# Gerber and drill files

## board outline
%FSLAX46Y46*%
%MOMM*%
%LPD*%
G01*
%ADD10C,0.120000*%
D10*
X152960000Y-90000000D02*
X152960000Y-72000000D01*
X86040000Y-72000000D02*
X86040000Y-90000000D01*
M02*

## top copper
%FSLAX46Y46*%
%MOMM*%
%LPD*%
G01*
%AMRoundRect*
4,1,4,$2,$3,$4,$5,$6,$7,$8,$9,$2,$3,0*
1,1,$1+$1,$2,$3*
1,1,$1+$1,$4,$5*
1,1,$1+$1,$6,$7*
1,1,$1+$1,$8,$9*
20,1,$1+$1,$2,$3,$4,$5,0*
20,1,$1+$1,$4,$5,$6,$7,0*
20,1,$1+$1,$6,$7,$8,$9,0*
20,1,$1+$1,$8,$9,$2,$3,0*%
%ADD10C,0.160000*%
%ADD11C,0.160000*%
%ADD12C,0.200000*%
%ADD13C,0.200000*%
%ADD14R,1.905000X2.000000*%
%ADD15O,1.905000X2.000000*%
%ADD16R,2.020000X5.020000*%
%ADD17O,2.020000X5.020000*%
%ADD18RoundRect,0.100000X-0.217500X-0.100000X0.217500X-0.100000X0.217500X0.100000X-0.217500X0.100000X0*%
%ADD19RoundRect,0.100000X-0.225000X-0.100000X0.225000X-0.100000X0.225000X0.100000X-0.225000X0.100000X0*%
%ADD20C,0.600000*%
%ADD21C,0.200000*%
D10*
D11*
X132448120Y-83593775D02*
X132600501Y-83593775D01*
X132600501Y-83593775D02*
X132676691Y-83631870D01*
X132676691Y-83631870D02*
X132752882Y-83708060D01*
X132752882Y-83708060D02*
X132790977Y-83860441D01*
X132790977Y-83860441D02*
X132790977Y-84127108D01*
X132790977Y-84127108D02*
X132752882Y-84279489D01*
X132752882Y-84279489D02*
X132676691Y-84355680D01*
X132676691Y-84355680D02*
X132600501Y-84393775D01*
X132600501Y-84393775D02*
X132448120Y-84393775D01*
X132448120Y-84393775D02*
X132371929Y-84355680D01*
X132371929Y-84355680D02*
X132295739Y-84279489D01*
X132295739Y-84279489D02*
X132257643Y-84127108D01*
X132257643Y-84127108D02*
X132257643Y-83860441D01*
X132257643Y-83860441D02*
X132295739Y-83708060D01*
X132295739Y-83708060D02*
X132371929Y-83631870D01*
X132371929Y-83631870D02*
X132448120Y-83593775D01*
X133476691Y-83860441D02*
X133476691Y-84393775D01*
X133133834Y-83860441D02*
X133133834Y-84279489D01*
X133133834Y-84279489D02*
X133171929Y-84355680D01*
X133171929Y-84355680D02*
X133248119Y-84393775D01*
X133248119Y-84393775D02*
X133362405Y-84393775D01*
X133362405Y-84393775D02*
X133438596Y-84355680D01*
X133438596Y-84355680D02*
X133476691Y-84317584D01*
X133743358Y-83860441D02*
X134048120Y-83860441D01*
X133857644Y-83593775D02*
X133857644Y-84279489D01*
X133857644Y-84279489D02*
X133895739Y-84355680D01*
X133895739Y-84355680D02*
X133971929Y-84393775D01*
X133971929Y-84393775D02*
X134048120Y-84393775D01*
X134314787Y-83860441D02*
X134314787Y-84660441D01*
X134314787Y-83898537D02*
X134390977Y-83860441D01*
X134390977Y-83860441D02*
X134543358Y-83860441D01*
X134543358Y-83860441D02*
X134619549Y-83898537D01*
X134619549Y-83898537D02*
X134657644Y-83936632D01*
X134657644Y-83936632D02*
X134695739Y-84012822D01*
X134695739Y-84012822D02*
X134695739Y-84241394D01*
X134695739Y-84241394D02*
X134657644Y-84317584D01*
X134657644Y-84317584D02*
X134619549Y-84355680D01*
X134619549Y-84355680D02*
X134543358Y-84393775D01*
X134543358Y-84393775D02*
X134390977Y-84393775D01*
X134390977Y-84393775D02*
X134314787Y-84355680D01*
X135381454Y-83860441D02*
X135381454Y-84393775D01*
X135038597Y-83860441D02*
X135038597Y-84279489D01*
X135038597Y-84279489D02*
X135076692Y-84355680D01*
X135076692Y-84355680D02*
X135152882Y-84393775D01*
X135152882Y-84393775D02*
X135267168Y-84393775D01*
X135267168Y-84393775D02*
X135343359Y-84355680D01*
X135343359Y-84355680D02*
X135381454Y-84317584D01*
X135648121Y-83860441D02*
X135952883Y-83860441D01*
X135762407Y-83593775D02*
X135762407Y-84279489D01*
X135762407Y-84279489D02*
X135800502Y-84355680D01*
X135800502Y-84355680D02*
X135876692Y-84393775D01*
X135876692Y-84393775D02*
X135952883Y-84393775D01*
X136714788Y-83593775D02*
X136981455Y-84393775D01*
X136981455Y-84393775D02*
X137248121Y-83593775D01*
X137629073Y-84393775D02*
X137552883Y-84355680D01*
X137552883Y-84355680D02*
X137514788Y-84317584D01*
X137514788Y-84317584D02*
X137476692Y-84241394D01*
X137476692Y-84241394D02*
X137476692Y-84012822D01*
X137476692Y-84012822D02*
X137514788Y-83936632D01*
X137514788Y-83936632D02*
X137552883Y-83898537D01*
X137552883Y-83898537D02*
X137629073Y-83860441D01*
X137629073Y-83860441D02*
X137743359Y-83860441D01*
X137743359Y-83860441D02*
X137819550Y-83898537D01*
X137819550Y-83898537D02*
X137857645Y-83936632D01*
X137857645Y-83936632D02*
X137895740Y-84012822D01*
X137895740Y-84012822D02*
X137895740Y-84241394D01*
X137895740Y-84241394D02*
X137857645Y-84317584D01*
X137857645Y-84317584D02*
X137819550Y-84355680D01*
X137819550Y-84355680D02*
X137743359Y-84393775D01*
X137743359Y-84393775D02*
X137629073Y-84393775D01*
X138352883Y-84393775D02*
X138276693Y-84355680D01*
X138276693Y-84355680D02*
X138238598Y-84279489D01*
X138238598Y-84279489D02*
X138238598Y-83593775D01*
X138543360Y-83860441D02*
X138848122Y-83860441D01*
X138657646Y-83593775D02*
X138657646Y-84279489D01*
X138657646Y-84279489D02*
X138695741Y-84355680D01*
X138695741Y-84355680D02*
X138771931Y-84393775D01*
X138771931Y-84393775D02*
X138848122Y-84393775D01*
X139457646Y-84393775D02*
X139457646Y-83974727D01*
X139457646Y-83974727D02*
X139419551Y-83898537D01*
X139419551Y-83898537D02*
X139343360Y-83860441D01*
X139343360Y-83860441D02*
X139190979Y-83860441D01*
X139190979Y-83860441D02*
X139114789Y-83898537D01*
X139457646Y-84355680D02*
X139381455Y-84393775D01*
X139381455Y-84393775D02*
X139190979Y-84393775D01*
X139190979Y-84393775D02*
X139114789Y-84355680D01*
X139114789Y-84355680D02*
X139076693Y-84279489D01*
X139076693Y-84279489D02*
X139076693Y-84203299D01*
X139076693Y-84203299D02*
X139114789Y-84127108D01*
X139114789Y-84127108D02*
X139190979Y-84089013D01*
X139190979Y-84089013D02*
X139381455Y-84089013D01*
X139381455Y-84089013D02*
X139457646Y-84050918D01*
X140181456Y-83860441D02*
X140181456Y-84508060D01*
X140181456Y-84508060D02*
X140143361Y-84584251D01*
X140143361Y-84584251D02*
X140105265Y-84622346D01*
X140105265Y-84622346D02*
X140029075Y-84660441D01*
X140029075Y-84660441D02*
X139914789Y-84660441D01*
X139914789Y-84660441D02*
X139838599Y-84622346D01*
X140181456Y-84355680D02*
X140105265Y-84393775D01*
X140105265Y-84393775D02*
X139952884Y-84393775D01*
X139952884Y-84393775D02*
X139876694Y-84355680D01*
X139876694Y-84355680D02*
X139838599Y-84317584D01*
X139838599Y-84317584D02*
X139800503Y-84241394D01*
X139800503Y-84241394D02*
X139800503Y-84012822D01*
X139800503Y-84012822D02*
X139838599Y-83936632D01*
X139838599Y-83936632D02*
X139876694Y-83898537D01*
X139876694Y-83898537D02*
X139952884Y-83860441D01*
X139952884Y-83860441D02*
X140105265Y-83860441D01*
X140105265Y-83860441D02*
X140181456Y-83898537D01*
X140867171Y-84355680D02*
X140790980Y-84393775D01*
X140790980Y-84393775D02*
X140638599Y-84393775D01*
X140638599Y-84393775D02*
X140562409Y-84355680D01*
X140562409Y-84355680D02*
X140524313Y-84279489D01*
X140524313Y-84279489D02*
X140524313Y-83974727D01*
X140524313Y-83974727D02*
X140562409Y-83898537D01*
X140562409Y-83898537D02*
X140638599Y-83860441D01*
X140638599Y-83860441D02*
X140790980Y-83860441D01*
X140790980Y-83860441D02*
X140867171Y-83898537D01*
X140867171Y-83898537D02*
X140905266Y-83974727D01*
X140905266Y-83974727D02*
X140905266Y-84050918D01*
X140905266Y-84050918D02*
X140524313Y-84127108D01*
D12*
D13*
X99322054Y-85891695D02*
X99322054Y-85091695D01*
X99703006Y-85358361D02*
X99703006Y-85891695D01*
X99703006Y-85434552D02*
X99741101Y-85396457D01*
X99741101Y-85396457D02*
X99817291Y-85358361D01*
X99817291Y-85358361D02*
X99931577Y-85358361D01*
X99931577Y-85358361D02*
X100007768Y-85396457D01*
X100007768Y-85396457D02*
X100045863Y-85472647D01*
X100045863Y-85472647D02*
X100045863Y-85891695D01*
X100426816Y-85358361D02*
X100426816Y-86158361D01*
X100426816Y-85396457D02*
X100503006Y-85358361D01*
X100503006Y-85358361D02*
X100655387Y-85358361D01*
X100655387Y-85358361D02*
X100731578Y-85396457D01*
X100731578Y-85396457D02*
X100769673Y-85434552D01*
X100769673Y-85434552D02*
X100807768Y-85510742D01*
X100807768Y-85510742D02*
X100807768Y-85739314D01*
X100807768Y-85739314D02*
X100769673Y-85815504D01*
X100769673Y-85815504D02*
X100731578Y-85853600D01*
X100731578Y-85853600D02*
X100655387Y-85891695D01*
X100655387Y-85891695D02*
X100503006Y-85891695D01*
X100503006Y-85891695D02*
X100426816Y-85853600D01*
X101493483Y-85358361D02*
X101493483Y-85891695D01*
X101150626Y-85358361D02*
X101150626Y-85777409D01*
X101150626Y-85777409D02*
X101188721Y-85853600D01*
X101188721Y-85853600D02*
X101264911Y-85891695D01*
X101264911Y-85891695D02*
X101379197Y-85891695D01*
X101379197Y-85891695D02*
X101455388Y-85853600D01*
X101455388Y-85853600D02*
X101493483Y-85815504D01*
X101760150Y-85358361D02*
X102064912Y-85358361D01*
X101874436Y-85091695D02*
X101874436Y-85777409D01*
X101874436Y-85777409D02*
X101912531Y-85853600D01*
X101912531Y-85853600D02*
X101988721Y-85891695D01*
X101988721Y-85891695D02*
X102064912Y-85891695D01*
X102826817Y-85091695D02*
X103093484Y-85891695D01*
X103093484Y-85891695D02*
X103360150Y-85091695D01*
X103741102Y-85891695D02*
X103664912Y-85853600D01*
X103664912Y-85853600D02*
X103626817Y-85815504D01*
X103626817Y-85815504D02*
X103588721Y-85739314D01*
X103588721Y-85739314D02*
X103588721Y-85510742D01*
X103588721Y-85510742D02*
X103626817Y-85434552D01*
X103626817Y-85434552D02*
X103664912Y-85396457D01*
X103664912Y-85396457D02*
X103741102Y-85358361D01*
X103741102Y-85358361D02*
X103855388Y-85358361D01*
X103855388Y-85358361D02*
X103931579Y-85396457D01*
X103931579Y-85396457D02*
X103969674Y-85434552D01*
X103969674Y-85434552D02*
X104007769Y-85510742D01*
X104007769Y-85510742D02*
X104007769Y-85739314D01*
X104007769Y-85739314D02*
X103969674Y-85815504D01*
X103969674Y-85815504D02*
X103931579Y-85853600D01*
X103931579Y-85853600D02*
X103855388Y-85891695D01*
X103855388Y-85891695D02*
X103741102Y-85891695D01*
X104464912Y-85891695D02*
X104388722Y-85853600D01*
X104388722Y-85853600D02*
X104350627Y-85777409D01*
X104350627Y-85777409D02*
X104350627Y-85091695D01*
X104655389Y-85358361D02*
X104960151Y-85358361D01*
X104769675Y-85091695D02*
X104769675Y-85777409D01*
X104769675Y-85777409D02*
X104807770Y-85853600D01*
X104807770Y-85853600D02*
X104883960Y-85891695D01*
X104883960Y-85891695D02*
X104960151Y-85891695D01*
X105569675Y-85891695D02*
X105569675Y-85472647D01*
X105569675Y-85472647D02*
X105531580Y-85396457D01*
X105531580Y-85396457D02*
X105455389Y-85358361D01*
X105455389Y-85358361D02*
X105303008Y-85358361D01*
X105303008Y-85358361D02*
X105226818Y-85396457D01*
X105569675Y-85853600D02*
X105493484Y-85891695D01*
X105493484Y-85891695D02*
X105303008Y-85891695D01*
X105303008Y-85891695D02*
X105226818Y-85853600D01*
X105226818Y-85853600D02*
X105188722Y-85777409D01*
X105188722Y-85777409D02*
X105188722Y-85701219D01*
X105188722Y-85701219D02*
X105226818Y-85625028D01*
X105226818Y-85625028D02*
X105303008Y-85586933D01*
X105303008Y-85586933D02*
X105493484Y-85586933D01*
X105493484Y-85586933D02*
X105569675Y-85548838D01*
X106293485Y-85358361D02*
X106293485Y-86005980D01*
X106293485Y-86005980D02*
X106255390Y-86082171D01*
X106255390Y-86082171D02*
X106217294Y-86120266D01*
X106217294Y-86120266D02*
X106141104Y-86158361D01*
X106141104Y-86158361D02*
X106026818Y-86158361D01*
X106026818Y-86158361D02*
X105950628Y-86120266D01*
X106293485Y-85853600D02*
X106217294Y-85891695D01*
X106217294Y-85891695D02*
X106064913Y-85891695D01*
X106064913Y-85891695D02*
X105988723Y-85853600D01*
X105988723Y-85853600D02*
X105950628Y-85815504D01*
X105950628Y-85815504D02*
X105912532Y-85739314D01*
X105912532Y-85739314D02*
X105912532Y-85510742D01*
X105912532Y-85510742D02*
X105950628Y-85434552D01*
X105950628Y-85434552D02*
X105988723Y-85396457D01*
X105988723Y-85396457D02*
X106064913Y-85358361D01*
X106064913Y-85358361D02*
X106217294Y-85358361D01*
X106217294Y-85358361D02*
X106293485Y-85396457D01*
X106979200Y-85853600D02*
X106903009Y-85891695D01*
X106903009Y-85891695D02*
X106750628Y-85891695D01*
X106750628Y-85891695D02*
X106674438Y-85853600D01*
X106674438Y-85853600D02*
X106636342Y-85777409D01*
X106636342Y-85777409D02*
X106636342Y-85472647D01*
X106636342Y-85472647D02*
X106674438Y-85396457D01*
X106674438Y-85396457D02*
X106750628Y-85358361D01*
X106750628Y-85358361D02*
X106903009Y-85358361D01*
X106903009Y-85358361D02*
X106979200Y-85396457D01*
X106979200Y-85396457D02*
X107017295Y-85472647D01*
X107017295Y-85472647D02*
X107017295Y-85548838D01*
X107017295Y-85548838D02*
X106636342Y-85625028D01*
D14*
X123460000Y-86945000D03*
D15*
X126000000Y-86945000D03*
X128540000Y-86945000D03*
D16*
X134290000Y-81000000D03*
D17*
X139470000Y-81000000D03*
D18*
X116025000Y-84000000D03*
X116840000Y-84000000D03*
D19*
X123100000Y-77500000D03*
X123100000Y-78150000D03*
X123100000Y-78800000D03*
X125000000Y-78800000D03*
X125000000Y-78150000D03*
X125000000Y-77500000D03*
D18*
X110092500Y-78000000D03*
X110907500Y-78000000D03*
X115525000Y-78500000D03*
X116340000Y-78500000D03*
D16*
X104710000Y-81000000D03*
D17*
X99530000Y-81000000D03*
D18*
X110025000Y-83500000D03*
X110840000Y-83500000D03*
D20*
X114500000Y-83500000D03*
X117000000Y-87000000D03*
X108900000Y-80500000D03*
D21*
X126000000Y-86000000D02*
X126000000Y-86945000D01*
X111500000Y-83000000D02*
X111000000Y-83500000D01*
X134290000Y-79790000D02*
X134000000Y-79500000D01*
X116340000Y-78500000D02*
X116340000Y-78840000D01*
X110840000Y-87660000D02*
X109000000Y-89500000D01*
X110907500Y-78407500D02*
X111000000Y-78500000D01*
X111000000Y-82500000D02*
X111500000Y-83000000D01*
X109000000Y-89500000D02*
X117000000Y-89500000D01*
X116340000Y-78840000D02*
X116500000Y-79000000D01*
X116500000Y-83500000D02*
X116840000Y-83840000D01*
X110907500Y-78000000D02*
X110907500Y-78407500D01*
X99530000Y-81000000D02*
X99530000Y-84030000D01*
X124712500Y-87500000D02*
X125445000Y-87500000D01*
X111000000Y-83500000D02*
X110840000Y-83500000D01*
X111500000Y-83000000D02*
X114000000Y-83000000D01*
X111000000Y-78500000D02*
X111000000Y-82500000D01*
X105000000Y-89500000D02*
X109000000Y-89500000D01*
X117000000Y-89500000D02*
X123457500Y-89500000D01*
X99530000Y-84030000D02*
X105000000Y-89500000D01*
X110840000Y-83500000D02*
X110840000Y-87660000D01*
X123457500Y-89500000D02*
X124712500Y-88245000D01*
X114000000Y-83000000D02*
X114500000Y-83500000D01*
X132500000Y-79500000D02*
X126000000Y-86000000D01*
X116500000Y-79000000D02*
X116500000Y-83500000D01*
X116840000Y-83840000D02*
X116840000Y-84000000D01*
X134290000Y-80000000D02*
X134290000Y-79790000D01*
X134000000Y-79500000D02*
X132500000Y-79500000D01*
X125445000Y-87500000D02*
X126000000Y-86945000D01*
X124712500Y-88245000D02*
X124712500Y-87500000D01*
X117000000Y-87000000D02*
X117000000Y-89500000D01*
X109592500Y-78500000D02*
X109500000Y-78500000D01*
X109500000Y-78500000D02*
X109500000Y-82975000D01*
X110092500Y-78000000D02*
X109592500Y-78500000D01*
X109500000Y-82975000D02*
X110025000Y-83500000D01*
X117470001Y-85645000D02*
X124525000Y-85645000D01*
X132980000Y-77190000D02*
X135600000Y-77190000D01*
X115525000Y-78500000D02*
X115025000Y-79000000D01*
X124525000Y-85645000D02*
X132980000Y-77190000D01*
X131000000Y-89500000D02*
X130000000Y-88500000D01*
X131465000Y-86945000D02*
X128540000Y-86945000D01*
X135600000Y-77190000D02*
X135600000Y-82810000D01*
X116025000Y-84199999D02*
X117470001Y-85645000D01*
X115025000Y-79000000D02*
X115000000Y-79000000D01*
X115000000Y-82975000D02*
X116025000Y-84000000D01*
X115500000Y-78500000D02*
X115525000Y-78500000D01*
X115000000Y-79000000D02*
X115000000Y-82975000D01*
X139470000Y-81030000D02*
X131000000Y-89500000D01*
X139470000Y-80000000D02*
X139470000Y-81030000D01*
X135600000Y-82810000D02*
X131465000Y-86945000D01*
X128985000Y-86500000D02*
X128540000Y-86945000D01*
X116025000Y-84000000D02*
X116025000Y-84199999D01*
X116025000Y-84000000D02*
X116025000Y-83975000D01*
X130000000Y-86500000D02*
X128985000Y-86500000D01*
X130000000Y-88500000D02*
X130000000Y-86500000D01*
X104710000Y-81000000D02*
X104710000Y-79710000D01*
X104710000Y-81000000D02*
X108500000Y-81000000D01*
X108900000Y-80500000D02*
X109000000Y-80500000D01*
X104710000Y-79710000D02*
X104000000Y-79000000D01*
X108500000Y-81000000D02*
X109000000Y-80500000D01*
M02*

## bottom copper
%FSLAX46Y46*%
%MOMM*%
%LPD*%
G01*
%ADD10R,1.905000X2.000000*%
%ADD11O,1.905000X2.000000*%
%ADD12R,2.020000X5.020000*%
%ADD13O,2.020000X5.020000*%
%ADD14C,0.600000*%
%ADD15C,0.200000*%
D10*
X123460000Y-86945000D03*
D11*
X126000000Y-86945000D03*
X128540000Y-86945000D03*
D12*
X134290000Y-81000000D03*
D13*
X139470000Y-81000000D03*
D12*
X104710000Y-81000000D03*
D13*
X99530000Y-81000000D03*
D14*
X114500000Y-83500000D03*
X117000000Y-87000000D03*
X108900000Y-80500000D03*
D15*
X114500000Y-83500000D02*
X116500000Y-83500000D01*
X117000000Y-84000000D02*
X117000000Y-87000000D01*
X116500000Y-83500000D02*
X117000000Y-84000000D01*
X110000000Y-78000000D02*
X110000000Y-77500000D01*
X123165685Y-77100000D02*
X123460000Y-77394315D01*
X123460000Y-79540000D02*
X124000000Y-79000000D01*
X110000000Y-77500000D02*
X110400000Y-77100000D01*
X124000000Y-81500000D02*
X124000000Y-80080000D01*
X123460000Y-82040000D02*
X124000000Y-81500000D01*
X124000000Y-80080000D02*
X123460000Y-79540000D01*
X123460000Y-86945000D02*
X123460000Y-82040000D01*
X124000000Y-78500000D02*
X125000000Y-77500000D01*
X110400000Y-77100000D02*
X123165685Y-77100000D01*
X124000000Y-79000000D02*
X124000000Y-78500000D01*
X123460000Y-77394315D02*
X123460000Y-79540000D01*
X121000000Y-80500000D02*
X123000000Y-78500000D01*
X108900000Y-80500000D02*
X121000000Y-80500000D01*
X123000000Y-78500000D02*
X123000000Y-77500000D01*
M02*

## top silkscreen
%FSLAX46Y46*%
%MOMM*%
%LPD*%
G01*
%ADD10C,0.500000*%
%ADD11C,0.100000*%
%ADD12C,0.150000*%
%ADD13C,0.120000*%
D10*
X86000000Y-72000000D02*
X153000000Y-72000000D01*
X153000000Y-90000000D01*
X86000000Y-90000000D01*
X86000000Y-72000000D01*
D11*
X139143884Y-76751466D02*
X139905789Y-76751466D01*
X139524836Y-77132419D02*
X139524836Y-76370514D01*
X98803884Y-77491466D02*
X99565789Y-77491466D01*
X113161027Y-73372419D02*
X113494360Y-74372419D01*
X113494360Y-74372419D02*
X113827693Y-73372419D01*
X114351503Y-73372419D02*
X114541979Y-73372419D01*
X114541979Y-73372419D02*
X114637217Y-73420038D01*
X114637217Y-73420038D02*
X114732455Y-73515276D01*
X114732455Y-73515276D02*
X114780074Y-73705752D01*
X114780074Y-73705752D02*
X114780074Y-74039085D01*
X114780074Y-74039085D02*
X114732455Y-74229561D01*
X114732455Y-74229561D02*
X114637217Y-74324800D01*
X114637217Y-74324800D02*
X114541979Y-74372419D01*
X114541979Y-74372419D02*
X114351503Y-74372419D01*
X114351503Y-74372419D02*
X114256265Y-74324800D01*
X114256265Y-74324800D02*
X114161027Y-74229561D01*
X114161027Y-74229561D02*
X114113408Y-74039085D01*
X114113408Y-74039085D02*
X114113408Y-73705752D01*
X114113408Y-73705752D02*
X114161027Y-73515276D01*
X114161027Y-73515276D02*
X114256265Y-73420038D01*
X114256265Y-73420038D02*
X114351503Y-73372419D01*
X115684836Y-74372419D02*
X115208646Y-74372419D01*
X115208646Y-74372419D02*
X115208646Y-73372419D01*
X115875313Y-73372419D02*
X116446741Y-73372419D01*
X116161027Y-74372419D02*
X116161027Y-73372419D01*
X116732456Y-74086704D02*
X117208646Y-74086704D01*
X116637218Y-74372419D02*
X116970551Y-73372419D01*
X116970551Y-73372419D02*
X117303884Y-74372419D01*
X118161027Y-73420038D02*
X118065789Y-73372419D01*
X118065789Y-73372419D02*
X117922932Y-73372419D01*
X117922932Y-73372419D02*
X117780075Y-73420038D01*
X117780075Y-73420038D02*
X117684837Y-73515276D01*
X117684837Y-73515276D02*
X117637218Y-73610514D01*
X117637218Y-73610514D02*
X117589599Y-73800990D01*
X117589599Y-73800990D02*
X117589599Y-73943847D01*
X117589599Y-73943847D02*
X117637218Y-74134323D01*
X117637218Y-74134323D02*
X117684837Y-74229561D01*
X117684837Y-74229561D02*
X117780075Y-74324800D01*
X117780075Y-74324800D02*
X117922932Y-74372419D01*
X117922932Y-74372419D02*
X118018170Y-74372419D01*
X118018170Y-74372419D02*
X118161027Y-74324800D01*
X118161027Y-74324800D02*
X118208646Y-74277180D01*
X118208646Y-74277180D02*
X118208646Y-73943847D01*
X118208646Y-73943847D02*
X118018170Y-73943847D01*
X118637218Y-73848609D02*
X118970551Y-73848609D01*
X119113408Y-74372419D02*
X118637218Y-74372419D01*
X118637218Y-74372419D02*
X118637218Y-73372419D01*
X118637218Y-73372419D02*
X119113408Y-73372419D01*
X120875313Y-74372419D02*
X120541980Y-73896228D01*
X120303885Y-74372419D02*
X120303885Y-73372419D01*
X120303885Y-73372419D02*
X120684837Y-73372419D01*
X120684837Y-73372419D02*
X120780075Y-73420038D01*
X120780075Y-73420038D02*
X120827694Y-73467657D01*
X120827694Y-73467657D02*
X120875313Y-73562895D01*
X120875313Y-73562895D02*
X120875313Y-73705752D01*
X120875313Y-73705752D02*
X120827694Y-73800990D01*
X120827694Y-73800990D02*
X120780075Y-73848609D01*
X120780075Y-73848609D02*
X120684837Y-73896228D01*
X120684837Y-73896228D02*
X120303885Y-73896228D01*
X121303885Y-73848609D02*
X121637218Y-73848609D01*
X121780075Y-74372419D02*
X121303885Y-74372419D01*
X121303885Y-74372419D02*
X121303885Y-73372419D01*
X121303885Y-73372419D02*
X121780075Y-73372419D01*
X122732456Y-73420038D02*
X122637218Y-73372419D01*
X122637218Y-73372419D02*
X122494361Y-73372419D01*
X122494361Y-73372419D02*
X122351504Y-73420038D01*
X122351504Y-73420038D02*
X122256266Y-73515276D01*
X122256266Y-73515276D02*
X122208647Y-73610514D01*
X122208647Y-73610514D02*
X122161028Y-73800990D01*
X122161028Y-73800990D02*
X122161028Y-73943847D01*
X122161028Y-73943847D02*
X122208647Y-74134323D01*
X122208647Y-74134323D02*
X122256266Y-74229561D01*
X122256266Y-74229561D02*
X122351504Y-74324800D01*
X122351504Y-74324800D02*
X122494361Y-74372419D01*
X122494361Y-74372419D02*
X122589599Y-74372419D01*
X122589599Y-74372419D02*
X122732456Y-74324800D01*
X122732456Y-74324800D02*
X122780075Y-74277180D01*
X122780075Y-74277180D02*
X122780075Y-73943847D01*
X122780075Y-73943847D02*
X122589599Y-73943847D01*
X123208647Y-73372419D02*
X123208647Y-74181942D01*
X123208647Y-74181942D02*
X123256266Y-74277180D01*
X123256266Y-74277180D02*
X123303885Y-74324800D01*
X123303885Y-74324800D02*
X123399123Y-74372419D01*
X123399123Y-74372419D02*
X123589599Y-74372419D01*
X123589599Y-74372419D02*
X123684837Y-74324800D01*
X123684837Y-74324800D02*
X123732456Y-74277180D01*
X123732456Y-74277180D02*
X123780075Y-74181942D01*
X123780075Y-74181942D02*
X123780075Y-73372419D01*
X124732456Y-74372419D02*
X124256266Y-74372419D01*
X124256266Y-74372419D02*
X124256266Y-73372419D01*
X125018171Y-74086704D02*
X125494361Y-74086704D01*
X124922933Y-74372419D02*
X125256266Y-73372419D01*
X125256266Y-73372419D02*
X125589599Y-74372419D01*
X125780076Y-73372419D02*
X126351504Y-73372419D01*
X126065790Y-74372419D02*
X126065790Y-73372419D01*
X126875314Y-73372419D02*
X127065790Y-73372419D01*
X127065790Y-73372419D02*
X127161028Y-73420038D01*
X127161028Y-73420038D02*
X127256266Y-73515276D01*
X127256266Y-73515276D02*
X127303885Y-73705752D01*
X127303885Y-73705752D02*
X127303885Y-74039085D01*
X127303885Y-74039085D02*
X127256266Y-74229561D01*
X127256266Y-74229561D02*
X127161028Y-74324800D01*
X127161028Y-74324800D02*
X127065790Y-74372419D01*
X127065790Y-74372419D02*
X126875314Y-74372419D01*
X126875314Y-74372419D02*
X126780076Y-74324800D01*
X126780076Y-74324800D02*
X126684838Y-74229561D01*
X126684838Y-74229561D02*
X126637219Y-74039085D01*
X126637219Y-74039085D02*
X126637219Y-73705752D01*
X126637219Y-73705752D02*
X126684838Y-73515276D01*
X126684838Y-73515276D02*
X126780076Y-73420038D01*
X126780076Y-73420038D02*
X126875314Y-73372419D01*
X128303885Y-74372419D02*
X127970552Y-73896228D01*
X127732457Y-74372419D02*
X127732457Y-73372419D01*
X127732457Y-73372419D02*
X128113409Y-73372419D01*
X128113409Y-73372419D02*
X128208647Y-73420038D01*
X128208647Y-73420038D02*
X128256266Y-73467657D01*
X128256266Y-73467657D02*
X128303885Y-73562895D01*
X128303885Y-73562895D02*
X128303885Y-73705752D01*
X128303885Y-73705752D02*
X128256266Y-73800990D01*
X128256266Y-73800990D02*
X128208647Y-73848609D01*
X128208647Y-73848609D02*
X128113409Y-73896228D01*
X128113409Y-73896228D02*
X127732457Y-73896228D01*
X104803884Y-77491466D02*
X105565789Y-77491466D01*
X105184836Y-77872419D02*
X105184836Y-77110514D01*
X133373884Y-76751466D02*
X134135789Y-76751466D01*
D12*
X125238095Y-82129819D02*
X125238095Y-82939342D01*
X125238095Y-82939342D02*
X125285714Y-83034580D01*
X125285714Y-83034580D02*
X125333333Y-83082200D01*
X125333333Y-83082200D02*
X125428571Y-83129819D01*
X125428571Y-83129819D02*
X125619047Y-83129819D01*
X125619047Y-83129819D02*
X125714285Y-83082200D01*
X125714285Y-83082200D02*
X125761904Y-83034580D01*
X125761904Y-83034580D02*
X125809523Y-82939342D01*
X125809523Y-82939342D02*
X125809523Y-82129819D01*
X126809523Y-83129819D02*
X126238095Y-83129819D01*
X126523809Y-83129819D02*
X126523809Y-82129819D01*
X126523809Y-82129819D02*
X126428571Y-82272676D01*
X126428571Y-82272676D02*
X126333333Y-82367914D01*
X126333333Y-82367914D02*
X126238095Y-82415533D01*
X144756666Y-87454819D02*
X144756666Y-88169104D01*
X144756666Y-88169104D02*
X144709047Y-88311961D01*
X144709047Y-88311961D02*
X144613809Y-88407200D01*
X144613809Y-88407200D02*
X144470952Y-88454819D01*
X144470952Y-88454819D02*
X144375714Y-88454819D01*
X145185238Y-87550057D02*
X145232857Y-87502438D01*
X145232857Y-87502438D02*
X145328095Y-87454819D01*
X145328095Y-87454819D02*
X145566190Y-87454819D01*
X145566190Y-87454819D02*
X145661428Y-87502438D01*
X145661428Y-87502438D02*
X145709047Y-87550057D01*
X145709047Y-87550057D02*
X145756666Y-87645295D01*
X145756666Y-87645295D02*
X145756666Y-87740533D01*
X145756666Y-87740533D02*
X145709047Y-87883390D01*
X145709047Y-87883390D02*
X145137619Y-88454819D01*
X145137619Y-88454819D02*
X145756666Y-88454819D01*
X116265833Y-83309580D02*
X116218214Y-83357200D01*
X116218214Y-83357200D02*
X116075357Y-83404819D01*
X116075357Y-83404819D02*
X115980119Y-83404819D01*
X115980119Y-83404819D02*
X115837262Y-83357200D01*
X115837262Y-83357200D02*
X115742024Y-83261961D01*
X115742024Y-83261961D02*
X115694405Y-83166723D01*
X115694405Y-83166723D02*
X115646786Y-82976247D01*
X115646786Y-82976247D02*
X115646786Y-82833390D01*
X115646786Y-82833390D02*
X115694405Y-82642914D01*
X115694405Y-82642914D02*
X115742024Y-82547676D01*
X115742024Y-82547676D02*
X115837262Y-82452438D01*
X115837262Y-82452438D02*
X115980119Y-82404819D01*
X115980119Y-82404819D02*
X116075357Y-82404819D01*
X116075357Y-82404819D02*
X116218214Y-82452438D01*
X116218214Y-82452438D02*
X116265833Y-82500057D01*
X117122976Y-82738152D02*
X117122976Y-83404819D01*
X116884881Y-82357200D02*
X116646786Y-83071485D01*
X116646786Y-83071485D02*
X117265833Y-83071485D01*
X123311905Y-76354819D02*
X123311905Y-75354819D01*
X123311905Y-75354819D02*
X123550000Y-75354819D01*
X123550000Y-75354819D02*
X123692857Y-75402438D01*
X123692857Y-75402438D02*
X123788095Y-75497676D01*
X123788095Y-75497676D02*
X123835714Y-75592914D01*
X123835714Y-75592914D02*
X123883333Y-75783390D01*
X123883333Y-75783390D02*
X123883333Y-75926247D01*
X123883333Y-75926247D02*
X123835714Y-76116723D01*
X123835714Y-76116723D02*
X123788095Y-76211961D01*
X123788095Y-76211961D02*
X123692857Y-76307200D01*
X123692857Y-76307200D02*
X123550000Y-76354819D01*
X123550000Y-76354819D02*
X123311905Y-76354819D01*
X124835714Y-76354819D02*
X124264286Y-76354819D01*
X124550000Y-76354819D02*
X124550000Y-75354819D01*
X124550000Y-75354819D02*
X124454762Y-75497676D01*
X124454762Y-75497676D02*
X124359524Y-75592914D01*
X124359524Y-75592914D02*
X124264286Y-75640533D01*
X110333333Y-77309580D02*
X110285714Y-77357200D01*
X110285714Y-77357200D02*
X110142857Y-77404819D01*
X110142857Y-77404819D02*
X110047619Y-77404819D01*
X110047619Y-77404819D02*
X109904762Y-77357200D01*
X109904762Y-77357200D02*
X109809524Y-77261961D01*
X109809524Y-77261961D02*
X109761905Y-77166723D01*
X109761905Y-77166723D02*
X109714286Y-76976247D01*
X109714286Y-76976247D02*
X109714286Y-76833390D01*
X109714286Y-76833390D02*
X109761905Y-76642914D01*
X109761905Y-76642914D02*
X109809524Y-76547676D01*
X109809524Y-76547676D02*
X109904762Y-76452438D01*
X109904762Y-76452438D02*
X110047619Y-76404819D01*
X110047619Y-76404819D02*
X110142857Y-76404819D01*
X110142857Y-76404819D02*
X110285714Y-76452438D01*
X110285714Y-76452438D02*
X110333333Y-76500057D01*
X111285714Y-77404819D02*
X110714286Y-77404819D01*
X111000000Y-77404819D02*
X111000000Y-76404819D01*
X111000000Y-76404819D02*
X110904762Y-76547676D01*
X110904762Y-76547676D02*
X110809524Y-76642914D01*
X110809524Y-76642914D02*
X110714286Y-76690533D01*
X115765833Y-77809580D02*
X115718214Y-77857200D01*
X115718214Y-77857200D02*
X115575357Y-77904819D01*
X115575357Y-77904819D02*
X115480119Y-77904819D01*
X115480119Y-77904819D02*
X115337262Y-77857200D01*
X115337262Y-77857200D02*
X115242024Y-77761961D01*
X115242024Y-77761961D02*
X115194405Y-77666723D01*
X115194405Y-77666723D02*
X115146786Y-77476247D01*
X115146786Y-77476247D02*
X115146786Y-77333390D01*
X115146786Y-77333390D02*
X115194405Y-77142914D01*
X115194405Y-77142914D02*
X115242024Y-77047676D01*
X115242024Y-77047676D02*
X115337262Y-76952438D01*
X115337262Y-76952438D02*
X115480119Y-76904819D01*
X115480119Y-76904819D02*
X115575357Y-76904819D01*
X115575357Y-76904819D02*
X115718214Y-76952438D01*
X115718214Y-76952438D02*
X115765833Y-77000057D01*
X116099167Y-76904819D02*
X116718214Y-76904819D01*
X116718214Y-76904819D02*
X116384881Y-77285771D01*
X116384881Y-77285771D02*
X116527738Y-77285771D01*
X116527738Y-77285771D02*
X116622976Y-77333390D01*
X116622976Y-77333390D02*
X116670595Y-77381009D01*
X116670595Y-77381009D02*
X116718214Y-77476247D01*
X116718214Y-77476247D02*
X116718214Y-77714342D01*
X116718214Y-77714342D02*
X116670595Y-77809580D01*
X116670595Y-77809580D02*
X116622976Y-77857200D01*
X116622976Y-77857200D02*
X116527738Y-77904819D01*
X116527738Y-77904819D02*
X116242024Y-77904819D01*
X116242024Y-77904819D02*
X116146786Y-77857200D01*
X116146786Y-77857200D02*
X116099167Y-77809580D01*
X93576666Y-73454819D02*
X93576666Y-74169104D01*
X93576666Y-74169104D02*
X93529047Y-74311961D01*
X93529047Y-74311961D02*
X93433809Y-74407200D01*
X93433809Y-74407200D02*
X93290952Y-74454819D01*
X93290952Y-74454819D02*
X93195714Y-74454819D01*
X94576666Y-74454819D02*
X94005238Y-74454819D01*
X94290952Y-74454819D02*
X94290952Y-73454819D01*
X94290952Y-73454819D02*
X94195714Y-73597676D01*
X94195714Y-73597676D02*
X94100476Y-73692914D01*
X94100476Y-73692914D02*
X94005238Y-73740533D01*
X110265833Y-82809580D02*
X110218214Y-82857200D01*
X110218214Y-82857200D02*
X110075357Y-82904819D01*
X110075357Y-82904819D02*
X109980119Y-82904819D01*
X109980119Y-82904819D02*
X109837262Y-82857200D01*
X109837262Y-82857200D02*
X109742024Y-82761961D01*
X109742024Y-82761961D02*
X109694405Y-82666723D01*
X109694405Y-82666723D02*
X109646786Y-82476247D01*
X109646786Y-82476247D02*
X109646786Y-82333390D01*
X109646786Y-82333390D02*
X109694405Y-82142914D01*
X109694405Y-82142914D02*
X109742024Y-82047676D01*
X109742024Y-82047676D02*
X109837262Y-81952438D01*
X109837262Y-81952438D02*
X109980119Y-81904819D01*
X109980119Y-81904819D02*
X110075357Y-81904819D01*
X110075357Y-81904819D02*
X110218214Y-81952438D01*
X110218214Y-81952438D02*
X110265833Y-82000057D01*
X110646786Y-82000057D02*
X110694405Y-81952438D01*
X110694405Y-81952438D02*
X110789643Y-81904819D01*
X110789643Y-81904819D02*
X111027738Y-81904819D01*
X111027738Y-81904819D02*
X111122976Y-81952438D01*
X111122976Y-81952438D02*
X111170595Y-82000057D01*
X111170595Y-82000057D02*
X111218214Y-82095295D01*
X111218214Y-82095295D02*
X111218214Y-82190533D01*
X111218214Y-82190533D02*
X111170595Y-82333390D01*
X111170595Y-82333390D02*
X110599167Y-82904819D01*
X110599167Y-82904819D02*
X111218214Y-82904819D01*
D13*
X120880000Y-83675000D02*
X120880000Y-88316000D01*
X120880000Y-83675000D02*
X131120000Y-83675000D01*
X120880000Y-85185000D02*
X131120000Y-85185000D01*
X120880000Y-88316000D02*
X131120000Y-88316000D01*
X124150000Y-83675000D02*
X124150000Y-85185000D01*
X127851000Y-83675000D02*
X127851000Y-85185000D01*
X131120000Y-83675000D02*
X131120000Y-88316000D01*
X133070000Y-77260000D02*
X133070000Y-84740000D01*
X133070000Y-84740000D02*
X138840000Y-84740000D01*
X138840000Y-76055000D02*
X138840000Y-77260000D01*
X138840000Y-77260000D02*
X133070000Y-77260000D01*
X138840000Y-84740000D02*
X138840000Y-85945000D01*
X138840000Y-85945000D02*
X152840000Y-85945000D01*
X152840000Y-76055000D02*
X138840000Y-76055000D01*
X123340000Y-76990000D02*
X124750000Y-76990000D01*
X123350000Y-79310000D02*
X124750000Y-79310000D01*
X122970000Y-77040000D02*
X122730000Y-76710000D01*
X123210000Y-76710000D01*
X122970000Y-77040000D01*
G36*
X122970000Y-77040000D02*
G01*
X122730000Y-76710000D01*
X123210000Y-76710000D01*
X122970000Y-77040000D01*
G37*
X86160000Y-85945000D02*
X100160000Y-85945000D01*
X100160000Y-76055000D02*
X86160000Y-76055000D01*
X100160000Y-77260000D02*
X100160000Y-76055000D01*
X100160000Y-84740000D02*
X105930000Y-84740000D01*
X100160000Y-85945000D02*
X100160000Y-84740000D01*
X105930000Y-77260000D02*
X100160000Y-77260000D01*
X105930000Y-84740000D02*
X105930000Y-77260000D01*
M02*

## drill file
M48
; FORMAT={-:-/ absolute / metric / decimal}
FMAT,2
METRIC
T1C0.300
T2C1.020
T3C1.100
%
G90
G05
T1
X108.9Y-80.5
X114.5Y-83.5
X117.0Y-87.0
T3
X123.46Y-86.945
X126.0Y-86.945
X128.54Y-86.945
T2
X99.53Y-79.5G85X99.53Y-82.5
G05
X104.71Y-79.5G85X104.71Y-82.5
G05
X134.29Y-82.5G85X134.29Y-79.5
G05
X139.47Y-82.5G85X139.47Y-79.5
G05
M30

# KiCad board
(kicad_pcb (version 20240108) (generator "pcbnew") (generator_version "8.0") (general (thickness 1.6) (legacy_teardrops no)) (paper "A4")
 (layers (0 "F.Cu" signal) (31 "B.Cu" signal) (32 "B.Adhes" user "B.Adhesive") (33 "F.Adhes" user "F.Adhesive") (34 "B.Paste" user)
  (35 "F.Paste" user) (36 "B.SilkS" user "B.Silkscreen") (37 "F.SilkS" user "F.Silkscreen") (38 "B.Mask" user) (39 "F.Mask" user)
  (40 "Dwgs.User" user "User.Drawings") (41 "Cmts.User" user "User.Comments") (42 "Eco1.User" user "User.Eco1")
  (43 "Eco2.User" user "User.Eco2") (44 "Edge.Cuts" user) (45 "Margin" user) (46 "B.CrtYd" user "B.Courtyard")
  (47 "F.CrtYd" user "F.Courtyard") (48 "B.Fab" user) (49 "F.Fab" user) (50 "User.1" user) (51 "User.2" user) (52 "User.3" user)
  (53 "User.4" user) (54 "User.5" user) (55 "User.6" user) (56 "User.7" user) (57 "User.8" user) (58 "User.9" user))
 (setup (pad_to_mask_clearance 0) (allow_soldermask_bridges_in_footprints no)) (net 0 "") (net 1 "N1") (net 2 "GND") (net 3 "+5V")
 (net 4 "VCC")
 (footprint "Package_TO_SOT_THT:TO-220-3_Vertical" (layer "F.Cu") (at 123.46 86.945)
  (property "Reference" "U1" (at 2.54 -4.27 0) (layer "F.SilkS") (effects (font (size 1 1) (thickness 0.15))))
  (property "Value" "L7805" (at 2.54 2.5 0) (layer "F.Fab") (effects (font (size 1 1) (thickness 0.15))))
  (fp_line (start -2.58 -3.27) (end -2.58 1.371) (stroke (width 0.12) (type solid)) (layer "F.SilkS"))
  (fp_line (start -2.58 -3.27) (end 7.66 -3.27) (stroke (width 0.12) (type solid)) (layer "F.SilkS"))
  (fp_line (start -2.58 -1.76) (end 7.66 -1.76) (stroke (width 0.12) (type solid)) (layer "F.SilkS"))
  (fp_line (start -2.58 1.371) (end 7.66 1.371) (stroke (width 0.12) (type solid)) (layer "F.SilkS"))
  (fp_line (start 0.69 -3.27) (end 0.69 -1.76) (stroke (width 0.12) (type solid)) (layer "F.SilkS"))
  (fp_line (start 4.391 -3.27) (end 4.391 -1.76) (stroke (width 0.12) (type solid)) (layer "F.SilkS"))
  (fp_line (start 7.66 -3.27) (end 7.66 1.371) (stroke (width 0.12) (type solid)) (layer "F.SilkS"))
  (pad "1" thru_hole rect (at 0 0) (size 1.905 2) (drill 1.1) (layers "*.Cu" "*.Mask") (remove_unused_layers no) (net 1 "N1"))
  (pad "2" thru_hole oval (at 2.54 0) (size 1.905 2) (drill 1.1) (layers "*.Cu" "*.Mask") (remove_unused_layers no) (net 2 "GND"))
  (pad "3" thru_hole oval (at 5.08 0) (size 1.905 2) (drill 1.1) (layers "*.Cu" "*.Mask") (remove_unused_layers no) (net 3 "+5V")))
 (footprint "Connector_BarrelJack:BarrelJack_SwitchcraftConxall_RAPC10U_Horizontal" (layer "F.Cu") (at 134.29 81 180)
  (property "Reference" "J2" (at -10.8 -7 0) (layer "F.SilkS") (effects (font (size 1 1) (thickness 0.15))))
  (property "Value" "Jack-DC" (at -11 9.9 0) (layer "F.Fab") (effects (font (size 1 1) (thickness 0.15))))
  (fp_line (start 1.22 3.74) (end 1.22 -3.74) (stroke (width 0.12) (type solid)) (layer "F.SilkS"))
  (fp_line (start 1.22 -3.74) (end -4.55 -3.74) (stroke (width 0.12) (type solid)) (layer "F.SilkS"))
  (fp_line (start -4.55 4.945) (end -4.55 3.74) (stroke (width 0.12) (type solid)) (layer "F.SilkS"))
  (fp_line (start -4.55 3.74) (end 1.22 3.74) (stroke (width 0.12) (type solid)) (layer "F.SilkS"))
  (fp_line (start -4.55 -3.74) (end -4.55 -4.945) (stroke (width 0.12) (type solid)) (layer "F.SilkS"))
  (fp_line (start -4.55 -4.945) (end -18.55 -4.945) (stroke (width 0.12) (type solid)) (layer "F.SilkS"))
  (fp_line (start -18.55 4.945) (end -4.55 4.945) (stroke (width 0.12) (type solid)) (layer "F.SilkS"))
  (fp_line (start -18.67 -9) (end -18.67 9) (stroke (width 0.12) (type solid)) (layer "Edge.Cuts"))
  (pad "1" thru_hole rect (at 0 0 180) (size 2.02 5.02) (drill oval 1.02 4.02) (layers "*.Cu" "*.Mask") (remove_unused_layers no)
   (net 2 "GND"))
  (pad "2" thru_hole oval (at -5.18 0 180) (size 2.02 5.02) (drill oval 1.02 4.02) (layers "*.Cu" "*.Mask") (remove_unused_layers no)
   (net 3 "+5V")))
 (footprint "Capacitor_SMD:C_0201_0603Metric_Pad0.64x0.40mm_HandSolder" (layer "F.Cu") (at 116.4325 84)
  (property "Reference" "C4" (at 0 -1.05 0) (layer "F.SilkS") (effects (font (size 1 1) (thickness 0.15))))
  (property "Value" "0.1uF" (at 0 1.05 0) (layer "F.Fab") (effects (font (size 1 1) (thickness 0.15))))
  (pad "" smd roundrect (at -0.4325 0) (size 0.458 0.36) (layers "F.Paste") (roundrect_rratio 0.25))
  (pad "" smd roundrect (at 0.4325 0) (size 0.458 0.36) (layers "F.Paste") (roundrect_rratio 0.25))
  (pad "1" smd roundrect (at -0.4075 0) (size 0.635 0.4) (layers "F.Cu" "F.Mask") (roundrect_rratio 0.25) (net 3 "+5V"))
  (pad "2" smd roundrect (at 0.4075 0) (size 0.635 0.4) (layers "F.Cu" "F.Mask") (roundrect_rratio 0.25) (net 2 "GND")))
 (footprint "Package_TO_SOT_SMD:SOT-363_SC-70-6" (layer "F.Cu") (at 124.05 78.15)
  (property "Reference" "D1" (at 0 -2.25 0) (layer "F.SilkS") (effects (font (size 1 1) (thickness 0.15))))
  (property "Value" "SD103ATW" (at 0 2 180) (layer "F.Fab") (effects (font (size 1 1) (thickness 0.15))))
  (fp_line (start -0.71 -1.16) (end 0.7 -1.16) (stroke (width 0.12) (type solid)) (layer "F.SilkS"))
  (fp_line (start -0.7 1.16) (end 0.7 1.16) (stroke (width 0.12) (type solid)) (layer "F.SilkS"))
  (fp_poly
   (pts (xy -1.08 -1.11) (xy -1.32 -1.44) (xy -0.84 -1.44) (xy -1.08 -1.11)) (stroke (width 0.12) (type solid)) (fill solid)
   (layer "F.SilkS"))
  (pad "1" smd roundrect (at -0.95 -0.65) (size 0.65 0.4) (layers "F.Cu" "F.Paste" "F.Mask") (roundrect_rratio 0.25) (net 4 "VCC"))
  (pad "2" smd roundrect (at -0.95 0) (size 0.65 0.4) (layers "F.Cu" "F.Paste" "F.Mask") (roundrect_rratio 0.25))
  (pad "3" smd roundrect (at -0.95 0.65) (size 0.65 0.4) (layers "F.Cu" "F.Paste" "F.Mask") (roundrect_rratio 0.25))
  (pad "4" smd roundrect (at 0.95 0.65) (size 0.65 0.4) (layers "F.Cu" "F.Paste" "F.Mask") (roundrect_rratio 0.25))
  (pad "5" smd roundrect (at 0.95 0) (size 0.65 0.4) (layers "F.Cu" "F.Paste" "F.Mask") (roundrect_rratio 0.25))
  (pad "6" smd roundrect (at 0.95 -0.65) (size 0.65 0.4) (layers "F.Cu" "F.Paste" "F.Mask") (roundrect_rratio 0.25) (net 1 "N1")))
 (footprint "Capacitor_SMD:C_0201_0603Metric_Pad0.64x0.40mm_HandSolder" (layer "F.Cu") (at 110.5 78)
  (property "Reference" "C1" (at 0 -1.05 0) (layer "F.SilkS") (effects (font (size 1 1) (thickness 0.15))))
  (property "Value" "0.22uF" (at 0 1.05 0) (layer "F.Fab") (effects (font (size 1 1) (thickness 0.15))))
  (pad "" smd roundrect (at -0.4325 0) (size 0.458 0.36) (layers "F.Paste") (roundrect_rratio 0.25))
  (pad "" smd roundrect (at 0.4325 0) (size 0.458 0.36) (layers "F.Paste") (roundrect_rratio 0.25))
  (pad "1" smd roundrect (at -0.4075 0) (size 0.635 0.4) (layers "F.Cu" "F.Mask") (roundrect_rratio 0.25) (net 1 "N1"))
  (pad "2" smd roundrect (at 0.4075 0) (size 0.635 0.4) (layers "F.Cu" "F.Mask") (roundrect_rratio 0.25) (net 2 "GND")))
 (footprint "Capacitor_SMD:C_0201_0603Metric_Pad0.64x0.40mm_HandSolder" (layer "F.Cu") (at 115.9325 78.5)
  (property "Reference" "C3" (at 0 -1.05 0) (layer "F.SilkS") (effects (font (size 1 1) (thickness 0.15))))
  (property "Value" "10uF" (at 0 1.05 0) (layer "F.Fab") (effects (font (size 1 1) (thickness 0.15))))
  (pad "" smd roundrect (at -0.4325 0) (size 0.458 0.36) (layers "F.Paste") (roundrect_rratio 0.25))
  (pad "" smd roundrect (at 0.4325 0) (size 0.458 0.36) (layers "F.Paste") (roundrect_rratio 0.25))
  (pad "1" smd roundrect (at -0.4075 0) (size 0.635 0.4) (layers "F.Cu" "F.Mask") (roundrect_rratio 0.25) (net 3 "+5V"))
  (pad "2" smd roundrect (at 0.4075 0) (size 0.635 0.4) (layers "F.Cu" "F.Mask") (roundrect_rratio 0.25) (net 2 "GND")))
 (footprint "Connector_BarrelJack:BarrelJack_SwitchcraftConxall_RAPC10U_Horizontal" (layer "F.Cu") (at 104.71 81)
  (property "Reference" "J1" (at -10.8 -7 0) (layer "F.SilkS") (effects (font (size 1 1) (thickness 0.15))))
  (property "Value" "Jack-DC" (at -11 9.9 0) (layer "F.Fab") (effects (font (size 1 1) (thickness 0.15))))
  (fp_line (start -18.55 4.945) (end -4.55 4.945) (stroke (width 0.12) (type solid)) (layer "F.SilkS"))
  (fp_line (start -4.55 -4.945) (end -18.55 -4.945) (stroke (width 0.12) (type solid)) (layer "F.SilkS"))
  (fp_line (start -4.55 -3.74) (end -4.55 -4.945) (stroke (width 0.12) (type solid)) (layer "F.SilkS"))
  (fp_line (start -4.55 3.74) (end 1.22 3.74) (stroke (width 0.12) (type solid)) (layer "F.SilkS"))
  (fp_line (start -4.55 4.945) (end -4.55 3.74) (stroke (width 0.12) (type solid)) (layer "F.SilkS"))
  (fp_line (start 1.22 -3.74) (end -4.55 -3.74) (stroke (width 0.12) (type solid)) (layer "F.SilkS"))
  (fp_line (start 1.22 3.74) (end 1.22 -3.74) (stroke (width 0.12) (type solid)) (layer "F.SilkS"))
  (fp_line (start -18.67 -9) (end -18.67 9) (stroke (width 0.12) (type solid)) (layer "Edge.Cuts"))
  (pad "1" thru_hole rect (at 0 0) (size 2.02 5.02) (drill oval 1.02 4.02) (layers "*.Cu" "*.Mask") (remove_unused_layers no) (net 4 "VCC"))
  (pad "2" thru_hole oval (at -5.18 0) (size 2.02 5.02) (drill oval 1.02 4.02) (layers "*.Cu" "*.Mask") (remove_unused_layers no)
   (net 2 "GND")))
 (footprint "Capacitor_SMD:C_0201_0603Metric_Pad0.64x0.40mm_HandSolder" (layer "F.Cu") (at 110.4325 83.5)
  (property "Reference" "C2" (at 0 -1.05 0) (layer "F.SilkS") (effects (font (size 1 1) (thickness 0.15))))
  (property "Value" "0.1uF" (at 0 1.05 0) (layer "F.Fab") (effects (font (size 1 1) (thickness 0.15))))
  (pad "" smd roundrect (at -0.4325 0) (size 0.458 0.36) (layers "F.Paste") (roundrect_rratio 0.25))
  (pad "" smd roundrect (at 0.4325 0) (size 0.458 0.36) (layers "F.Paste") (roundrect_rratio 0.25))
  (pad "1" smd roundrect (at -0.4075 0) (size 0.635 0.4) (layers "F.Cu" "F.Mask") (roundrect_rratio 0.25) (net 1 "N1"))
  (pad "2" smd roundrect (at 0.4075 0) (size 0.635 0.4) (layers "F.Cu" "F.Mask") (roundrect_rratio 0.25) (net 2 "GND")))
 (gr_rect (start 86 72) (end 153 90) (stroke (width 0.5) (type default)) (fill none) (layer "F.SilkS"))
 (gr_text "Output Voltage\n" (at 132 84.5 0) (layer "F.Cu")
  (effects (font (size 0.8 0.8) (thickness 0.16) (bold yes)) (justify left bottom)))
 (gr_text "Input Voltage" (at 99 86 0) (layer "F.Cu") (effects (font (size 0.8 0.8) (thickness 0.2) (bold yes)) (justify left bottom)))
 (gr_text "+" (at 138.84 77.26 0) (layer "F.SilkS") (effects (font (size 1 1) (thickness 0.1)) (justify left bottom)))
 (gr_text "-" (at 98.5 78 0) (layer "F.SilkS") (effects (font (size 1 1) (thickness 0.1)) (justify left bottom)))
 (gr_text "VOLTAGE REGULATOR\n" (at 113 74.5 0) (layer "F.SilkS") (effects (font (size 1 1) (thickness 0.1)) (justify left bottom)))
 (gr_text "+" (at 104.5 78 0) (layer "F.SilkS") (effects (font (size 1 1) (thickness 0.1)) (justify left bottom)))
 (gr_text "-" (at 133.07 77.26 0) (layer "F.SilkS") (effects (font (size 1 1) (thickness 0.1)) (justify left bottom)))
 (segment (start 126 86) (end 126 86.945) (width 0.2) (layer "F.Cu") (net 2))
 (segment (start 111.5 83) (end 111 83.5) (width 0.2) (layer "F.Cu") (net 2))
 (segment (start 134.29 79.79) (end 134 79.5) (width 0.2) (layer "F.Cu") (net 2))
 (segment (start 116.34 78.5) (end 116.34 78.84) (width 0.2) (layer "F.Cu") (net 2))
 (segment (start 110.84 87.66) (end 109 89.5) (width 0.2) (layer "F.Cu") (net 2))
 (segment (start 110.9075 78.4075) (end 111 78.5) (width 0.2) (layer "F.Cu") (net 2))
 (segment (start 111 82.5) (end 111.5 83) (width 0.2) (layer "F.Cu") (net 2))
 (segment (start 109 89.5) (end 117 89.5) (width 0.2) (layer "F.Cu") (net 2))
 (segment (start 116.34 78.84) (end 116.5 79) (width 0.2) (layer "F.Cu") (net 2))
 (segment (start 116.5 83.5) (end 116.84 83.84) (width 0.2) (layer "F.Cu") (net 2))
 (segment (start 110.9075 78) (end 110.9075 78.4075) (width 0.2) (layer "F.Cu") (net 2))
 (segment (start 99.53 81) (end 99.53 84.03) (width 0.2) (layer "F.Cu") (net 2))
 (segment (start 124.7125 87.5) (end 125.445 87.5) (width 0.2) (layer "F.Cu") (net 2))
 (segment (start 111 83.5) (end 110.84 83.5) (width 0.2) (layer "F.Cu") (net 2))
 (segment (start 111.5 83) (end 114 83) (width 0.2) (layer "F.Cu") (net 2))
 (segment (start 111 78.5) (end 111 82.5) (width 0.2) (layer "F.Cu") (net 2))
 (segment (start 105 89.5) (end 109 89.5) (width 0.2) (layer "F.Cu") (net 2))
 (segment (start 117 89.5) (end 123.4575 89.5) (width 0.2) (layer "F.Cu") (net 2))
 (segment (start 99.53 84.03) (end 105 89.5) (width 0.2) (layer "F.Cu") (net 2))
 (segment (start 110.84 83.5) (end 110.84 87.66) (width 0.2) (layer "F.Cu") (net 2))
 (segment (start 123.4575 89.5) (end 124.7125 88.245) (width 0.2) (layer "F.Cu") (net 2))
 (segment (start 114 83) (end 114.5 83.5) (width 0.2) (layer "F.Cu") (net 2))
 (segment (start 132.5 79.5) (end 126 86) (width 0.2) (layer "F.Cu") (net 2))
 (segment (start 116.5 79) (end 116.5 83.5) (width 0.2) (layer "F.Cu") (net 2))
 (segment (start 116.84 83.84) (end 116.84 84) (width 0.2) (layer "F.Cu") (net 2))
 (segment (start 134.29 80) (end 134.29 79.79) (width 0.2) (layer "F.Cu") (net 2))
 (segment (start 134 79.5) (end 132.5 79.5) (width 0.2) (layer "F.Cu") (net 2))
 (segment (start 125.445 87.5) (end 126 86.945) (width 0.2) (layer "F.Cu") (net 2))
 (segment (start 124.7125 88.245) (end 124.7125 87.5) (width 0.2) (layer "F.Cu") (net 2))
 (segment (start 117 87) (end 117 89.5) (width 0.2) (layer "F.Cu") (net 2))
 (via (at 114.5 83.5) (size 0.6) (drill 0.3) (layers "F.Cu" "B.Cu") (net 2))
 (via (at 117 87) (size 0.6) (drill 0.3) (layers "F.Cu" "B.Cu") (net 2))
 (segment (start 114.5 83.5) (end 116.5 83.5) (width 0.2) (layer "B.Cu") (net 2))
 (segment (start 117 84) (end 117 87) (width 0.2) (layer "B.Cu") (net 2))
 (segment (start 116.5 83.5) (end 117 84) (width 0.2) (layer "B.Cu") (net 2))
 (segment (start 109.5925 78.5) (end 109.5 78.5) (width 0.2) (layer "F.Cu") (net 1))
 (segment (start 109.5 78.5) (end 109.5 82.975) (width 0.2) (layer "F.Cu") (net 1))
 (segment (start 110.0925 78) (end 109.5925 78.5) (width 0.2) (layer "F.Cu") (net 1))
 (segment (start 109.5 82.975) (end 110.025 83.5) (width 0.2) (layer "F.Cu") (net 1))
 (segment (start 110 78) (end 110 77.5) (width 0.2) (layer "B.Cu") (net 1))
 (segment (start 123.165685 77.1) (end 123.46 77.394315) (width 0.2) (layer "B.Cu") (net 1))
 (segment (start 123.46 79.54) (end 124 79) (width 0.2) (layer "B.Cu") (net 1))
 (segment (start 110 77.5) (end 110.4 77.1) (width 0.2) (layer "B.Cu") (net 1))
 (segment (start 124 81.5) (end 124 80.08) (width 0.2) (layer "B.Cu") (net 1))
 (segment (start 123.46 82.04) (end 124 81.5) (width 0.2) (layer "B.Cu") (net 1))
 (segment (start 124 80.08) (end 123.46 79.54) (width 0.2) (layer "B.Cu") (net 1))
 (segment (start 123.46 86.945) (end 123.46 82.04) (width 0.2) (layer "B.Cu") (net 1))
 (segment (start 124 78.5) (end 125 77.5) (width 0.2) (layer "B.Cu") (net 1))
 (segment (start 110.4 77.1) (end 123.165685 77.1) (width 0.2) (layer "B.Cu") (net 1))
 (segment (start 124 79) (end 124 78.5) (width 0.2) (layer "B.Cu") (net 1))
 (segment (start 123.46 77.394315) (end 123.46 79.54) (width 0.2) (layer "B.Cu") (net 1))
 (segment (start 117.470001 85.645) (end 124.525 85.645) (width 0.2) (layer "F.Cu") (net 3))
 (segment (start 132.98 77.19) (end 135.6 77.19) (width 0.2) (layer "F.Cu") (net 3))
 (segment (start 115.525 78.5) (end 115.025 79) (width 0.2) (layer "F.Cu") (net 3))
 (segment (start 124.525 85.645) (end 132.98 77.19) (width 0.2) (layer "F.Cu") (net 3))
 (segment (start 131 89.5) (end 130 88.5) (width 0.2) (layer "F.Cu") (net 3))
 (segment (start 131.465 86.945) (end 128.54 86.945) (width 0.2) (layer "F.Cu") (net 3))
 (segment (start 135.6 77.19) (end 135.6 82.81) (width 0.2) (layer "F.Cu") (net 3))
 (segment (start 116.025 84.199999) (end 117.470001 85.645) (width 0.2) (layer "F.Cu") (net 3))
 (segment (start 115.025 79) (end 115 79) (width 0.2) (layer "F.Cu") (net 3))
 (segment (start 115 82.975) (end 116.025 84) (width 0.2) (layer "F.Cu") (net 3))
 (segment (start 115.5 78.5) (end 115.525 78.5) (width 0.2) (layer "F.Cu") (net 3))
 (segment (start 115 79) (end 115 82.975) (width 0.2) (layer "F.Cu") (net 3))
 (segment (start 139.47 81.03) (end 131 89.5) (width 0.2) (layer "F.Cu") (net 3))
 (segment (start 139.47 80) (end 139.47 81.03) (width 0.2) (layer "F.Cu") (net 3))
 (segment (start 135.6 82.81) (end 131.465 86.945) (width 0.2) (layer "F.Cu") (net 3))
 (segment (start 128.985 86.5) (end 128.54 86.945) (width 0.2) (layer "F.Cu") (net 3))
 (segment (start 116.025 84) (end 116.025 84.199999) (width 0.2) (layer "F.Cu") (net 3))
 (segment (start 116.025 84) (end 116.025 83.975) (width 0.2) (layer "F.Cu") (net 3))
 (segment (start 130 86.5) (end 128.985 86.5) (width 0.2) (layer "F.Cu") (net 3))
 (segment (start 130 88.5) (end 130 86.5) (width 0.2) (layer "F.Cu") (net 3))
 (segment (start 104.71 81) (end 104.71 79.71) (width 0.2) (layer "F.Cu") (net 4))
 (segment (start 104.71 81) (end 108.5 81) (width 0.2) (layer "F.Cu") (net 4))
 (segment (start 108.9 80.5) (end 109 80.5) (width 0.2) (layer "F.Cu") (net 4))
 (segment (start 104.71 79.71) (end 104 79) (width 0.2) (layer "F.Cu") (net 4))
 (segment (start 108.5 81) (end 109 80.5) (width 0.2) (layer "F.Cu") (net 4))
 (via (at 108.9 80.5) (size 0.6) (drill 0.3) (layers "F.Cu" "B.Cu") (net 4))
 (segment (start 121 80.5) (end 123 78.5) (width 0.2) (layer "B.Cu") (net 4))
 (segment (start 108.9 80.5) (end 121 80.5) (width 0.2) (layer "B.Cu") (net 4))
 (segment (start 123 78.5) (end 123 77.5) (width 0.2) (layer "B.Cu") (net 4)))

